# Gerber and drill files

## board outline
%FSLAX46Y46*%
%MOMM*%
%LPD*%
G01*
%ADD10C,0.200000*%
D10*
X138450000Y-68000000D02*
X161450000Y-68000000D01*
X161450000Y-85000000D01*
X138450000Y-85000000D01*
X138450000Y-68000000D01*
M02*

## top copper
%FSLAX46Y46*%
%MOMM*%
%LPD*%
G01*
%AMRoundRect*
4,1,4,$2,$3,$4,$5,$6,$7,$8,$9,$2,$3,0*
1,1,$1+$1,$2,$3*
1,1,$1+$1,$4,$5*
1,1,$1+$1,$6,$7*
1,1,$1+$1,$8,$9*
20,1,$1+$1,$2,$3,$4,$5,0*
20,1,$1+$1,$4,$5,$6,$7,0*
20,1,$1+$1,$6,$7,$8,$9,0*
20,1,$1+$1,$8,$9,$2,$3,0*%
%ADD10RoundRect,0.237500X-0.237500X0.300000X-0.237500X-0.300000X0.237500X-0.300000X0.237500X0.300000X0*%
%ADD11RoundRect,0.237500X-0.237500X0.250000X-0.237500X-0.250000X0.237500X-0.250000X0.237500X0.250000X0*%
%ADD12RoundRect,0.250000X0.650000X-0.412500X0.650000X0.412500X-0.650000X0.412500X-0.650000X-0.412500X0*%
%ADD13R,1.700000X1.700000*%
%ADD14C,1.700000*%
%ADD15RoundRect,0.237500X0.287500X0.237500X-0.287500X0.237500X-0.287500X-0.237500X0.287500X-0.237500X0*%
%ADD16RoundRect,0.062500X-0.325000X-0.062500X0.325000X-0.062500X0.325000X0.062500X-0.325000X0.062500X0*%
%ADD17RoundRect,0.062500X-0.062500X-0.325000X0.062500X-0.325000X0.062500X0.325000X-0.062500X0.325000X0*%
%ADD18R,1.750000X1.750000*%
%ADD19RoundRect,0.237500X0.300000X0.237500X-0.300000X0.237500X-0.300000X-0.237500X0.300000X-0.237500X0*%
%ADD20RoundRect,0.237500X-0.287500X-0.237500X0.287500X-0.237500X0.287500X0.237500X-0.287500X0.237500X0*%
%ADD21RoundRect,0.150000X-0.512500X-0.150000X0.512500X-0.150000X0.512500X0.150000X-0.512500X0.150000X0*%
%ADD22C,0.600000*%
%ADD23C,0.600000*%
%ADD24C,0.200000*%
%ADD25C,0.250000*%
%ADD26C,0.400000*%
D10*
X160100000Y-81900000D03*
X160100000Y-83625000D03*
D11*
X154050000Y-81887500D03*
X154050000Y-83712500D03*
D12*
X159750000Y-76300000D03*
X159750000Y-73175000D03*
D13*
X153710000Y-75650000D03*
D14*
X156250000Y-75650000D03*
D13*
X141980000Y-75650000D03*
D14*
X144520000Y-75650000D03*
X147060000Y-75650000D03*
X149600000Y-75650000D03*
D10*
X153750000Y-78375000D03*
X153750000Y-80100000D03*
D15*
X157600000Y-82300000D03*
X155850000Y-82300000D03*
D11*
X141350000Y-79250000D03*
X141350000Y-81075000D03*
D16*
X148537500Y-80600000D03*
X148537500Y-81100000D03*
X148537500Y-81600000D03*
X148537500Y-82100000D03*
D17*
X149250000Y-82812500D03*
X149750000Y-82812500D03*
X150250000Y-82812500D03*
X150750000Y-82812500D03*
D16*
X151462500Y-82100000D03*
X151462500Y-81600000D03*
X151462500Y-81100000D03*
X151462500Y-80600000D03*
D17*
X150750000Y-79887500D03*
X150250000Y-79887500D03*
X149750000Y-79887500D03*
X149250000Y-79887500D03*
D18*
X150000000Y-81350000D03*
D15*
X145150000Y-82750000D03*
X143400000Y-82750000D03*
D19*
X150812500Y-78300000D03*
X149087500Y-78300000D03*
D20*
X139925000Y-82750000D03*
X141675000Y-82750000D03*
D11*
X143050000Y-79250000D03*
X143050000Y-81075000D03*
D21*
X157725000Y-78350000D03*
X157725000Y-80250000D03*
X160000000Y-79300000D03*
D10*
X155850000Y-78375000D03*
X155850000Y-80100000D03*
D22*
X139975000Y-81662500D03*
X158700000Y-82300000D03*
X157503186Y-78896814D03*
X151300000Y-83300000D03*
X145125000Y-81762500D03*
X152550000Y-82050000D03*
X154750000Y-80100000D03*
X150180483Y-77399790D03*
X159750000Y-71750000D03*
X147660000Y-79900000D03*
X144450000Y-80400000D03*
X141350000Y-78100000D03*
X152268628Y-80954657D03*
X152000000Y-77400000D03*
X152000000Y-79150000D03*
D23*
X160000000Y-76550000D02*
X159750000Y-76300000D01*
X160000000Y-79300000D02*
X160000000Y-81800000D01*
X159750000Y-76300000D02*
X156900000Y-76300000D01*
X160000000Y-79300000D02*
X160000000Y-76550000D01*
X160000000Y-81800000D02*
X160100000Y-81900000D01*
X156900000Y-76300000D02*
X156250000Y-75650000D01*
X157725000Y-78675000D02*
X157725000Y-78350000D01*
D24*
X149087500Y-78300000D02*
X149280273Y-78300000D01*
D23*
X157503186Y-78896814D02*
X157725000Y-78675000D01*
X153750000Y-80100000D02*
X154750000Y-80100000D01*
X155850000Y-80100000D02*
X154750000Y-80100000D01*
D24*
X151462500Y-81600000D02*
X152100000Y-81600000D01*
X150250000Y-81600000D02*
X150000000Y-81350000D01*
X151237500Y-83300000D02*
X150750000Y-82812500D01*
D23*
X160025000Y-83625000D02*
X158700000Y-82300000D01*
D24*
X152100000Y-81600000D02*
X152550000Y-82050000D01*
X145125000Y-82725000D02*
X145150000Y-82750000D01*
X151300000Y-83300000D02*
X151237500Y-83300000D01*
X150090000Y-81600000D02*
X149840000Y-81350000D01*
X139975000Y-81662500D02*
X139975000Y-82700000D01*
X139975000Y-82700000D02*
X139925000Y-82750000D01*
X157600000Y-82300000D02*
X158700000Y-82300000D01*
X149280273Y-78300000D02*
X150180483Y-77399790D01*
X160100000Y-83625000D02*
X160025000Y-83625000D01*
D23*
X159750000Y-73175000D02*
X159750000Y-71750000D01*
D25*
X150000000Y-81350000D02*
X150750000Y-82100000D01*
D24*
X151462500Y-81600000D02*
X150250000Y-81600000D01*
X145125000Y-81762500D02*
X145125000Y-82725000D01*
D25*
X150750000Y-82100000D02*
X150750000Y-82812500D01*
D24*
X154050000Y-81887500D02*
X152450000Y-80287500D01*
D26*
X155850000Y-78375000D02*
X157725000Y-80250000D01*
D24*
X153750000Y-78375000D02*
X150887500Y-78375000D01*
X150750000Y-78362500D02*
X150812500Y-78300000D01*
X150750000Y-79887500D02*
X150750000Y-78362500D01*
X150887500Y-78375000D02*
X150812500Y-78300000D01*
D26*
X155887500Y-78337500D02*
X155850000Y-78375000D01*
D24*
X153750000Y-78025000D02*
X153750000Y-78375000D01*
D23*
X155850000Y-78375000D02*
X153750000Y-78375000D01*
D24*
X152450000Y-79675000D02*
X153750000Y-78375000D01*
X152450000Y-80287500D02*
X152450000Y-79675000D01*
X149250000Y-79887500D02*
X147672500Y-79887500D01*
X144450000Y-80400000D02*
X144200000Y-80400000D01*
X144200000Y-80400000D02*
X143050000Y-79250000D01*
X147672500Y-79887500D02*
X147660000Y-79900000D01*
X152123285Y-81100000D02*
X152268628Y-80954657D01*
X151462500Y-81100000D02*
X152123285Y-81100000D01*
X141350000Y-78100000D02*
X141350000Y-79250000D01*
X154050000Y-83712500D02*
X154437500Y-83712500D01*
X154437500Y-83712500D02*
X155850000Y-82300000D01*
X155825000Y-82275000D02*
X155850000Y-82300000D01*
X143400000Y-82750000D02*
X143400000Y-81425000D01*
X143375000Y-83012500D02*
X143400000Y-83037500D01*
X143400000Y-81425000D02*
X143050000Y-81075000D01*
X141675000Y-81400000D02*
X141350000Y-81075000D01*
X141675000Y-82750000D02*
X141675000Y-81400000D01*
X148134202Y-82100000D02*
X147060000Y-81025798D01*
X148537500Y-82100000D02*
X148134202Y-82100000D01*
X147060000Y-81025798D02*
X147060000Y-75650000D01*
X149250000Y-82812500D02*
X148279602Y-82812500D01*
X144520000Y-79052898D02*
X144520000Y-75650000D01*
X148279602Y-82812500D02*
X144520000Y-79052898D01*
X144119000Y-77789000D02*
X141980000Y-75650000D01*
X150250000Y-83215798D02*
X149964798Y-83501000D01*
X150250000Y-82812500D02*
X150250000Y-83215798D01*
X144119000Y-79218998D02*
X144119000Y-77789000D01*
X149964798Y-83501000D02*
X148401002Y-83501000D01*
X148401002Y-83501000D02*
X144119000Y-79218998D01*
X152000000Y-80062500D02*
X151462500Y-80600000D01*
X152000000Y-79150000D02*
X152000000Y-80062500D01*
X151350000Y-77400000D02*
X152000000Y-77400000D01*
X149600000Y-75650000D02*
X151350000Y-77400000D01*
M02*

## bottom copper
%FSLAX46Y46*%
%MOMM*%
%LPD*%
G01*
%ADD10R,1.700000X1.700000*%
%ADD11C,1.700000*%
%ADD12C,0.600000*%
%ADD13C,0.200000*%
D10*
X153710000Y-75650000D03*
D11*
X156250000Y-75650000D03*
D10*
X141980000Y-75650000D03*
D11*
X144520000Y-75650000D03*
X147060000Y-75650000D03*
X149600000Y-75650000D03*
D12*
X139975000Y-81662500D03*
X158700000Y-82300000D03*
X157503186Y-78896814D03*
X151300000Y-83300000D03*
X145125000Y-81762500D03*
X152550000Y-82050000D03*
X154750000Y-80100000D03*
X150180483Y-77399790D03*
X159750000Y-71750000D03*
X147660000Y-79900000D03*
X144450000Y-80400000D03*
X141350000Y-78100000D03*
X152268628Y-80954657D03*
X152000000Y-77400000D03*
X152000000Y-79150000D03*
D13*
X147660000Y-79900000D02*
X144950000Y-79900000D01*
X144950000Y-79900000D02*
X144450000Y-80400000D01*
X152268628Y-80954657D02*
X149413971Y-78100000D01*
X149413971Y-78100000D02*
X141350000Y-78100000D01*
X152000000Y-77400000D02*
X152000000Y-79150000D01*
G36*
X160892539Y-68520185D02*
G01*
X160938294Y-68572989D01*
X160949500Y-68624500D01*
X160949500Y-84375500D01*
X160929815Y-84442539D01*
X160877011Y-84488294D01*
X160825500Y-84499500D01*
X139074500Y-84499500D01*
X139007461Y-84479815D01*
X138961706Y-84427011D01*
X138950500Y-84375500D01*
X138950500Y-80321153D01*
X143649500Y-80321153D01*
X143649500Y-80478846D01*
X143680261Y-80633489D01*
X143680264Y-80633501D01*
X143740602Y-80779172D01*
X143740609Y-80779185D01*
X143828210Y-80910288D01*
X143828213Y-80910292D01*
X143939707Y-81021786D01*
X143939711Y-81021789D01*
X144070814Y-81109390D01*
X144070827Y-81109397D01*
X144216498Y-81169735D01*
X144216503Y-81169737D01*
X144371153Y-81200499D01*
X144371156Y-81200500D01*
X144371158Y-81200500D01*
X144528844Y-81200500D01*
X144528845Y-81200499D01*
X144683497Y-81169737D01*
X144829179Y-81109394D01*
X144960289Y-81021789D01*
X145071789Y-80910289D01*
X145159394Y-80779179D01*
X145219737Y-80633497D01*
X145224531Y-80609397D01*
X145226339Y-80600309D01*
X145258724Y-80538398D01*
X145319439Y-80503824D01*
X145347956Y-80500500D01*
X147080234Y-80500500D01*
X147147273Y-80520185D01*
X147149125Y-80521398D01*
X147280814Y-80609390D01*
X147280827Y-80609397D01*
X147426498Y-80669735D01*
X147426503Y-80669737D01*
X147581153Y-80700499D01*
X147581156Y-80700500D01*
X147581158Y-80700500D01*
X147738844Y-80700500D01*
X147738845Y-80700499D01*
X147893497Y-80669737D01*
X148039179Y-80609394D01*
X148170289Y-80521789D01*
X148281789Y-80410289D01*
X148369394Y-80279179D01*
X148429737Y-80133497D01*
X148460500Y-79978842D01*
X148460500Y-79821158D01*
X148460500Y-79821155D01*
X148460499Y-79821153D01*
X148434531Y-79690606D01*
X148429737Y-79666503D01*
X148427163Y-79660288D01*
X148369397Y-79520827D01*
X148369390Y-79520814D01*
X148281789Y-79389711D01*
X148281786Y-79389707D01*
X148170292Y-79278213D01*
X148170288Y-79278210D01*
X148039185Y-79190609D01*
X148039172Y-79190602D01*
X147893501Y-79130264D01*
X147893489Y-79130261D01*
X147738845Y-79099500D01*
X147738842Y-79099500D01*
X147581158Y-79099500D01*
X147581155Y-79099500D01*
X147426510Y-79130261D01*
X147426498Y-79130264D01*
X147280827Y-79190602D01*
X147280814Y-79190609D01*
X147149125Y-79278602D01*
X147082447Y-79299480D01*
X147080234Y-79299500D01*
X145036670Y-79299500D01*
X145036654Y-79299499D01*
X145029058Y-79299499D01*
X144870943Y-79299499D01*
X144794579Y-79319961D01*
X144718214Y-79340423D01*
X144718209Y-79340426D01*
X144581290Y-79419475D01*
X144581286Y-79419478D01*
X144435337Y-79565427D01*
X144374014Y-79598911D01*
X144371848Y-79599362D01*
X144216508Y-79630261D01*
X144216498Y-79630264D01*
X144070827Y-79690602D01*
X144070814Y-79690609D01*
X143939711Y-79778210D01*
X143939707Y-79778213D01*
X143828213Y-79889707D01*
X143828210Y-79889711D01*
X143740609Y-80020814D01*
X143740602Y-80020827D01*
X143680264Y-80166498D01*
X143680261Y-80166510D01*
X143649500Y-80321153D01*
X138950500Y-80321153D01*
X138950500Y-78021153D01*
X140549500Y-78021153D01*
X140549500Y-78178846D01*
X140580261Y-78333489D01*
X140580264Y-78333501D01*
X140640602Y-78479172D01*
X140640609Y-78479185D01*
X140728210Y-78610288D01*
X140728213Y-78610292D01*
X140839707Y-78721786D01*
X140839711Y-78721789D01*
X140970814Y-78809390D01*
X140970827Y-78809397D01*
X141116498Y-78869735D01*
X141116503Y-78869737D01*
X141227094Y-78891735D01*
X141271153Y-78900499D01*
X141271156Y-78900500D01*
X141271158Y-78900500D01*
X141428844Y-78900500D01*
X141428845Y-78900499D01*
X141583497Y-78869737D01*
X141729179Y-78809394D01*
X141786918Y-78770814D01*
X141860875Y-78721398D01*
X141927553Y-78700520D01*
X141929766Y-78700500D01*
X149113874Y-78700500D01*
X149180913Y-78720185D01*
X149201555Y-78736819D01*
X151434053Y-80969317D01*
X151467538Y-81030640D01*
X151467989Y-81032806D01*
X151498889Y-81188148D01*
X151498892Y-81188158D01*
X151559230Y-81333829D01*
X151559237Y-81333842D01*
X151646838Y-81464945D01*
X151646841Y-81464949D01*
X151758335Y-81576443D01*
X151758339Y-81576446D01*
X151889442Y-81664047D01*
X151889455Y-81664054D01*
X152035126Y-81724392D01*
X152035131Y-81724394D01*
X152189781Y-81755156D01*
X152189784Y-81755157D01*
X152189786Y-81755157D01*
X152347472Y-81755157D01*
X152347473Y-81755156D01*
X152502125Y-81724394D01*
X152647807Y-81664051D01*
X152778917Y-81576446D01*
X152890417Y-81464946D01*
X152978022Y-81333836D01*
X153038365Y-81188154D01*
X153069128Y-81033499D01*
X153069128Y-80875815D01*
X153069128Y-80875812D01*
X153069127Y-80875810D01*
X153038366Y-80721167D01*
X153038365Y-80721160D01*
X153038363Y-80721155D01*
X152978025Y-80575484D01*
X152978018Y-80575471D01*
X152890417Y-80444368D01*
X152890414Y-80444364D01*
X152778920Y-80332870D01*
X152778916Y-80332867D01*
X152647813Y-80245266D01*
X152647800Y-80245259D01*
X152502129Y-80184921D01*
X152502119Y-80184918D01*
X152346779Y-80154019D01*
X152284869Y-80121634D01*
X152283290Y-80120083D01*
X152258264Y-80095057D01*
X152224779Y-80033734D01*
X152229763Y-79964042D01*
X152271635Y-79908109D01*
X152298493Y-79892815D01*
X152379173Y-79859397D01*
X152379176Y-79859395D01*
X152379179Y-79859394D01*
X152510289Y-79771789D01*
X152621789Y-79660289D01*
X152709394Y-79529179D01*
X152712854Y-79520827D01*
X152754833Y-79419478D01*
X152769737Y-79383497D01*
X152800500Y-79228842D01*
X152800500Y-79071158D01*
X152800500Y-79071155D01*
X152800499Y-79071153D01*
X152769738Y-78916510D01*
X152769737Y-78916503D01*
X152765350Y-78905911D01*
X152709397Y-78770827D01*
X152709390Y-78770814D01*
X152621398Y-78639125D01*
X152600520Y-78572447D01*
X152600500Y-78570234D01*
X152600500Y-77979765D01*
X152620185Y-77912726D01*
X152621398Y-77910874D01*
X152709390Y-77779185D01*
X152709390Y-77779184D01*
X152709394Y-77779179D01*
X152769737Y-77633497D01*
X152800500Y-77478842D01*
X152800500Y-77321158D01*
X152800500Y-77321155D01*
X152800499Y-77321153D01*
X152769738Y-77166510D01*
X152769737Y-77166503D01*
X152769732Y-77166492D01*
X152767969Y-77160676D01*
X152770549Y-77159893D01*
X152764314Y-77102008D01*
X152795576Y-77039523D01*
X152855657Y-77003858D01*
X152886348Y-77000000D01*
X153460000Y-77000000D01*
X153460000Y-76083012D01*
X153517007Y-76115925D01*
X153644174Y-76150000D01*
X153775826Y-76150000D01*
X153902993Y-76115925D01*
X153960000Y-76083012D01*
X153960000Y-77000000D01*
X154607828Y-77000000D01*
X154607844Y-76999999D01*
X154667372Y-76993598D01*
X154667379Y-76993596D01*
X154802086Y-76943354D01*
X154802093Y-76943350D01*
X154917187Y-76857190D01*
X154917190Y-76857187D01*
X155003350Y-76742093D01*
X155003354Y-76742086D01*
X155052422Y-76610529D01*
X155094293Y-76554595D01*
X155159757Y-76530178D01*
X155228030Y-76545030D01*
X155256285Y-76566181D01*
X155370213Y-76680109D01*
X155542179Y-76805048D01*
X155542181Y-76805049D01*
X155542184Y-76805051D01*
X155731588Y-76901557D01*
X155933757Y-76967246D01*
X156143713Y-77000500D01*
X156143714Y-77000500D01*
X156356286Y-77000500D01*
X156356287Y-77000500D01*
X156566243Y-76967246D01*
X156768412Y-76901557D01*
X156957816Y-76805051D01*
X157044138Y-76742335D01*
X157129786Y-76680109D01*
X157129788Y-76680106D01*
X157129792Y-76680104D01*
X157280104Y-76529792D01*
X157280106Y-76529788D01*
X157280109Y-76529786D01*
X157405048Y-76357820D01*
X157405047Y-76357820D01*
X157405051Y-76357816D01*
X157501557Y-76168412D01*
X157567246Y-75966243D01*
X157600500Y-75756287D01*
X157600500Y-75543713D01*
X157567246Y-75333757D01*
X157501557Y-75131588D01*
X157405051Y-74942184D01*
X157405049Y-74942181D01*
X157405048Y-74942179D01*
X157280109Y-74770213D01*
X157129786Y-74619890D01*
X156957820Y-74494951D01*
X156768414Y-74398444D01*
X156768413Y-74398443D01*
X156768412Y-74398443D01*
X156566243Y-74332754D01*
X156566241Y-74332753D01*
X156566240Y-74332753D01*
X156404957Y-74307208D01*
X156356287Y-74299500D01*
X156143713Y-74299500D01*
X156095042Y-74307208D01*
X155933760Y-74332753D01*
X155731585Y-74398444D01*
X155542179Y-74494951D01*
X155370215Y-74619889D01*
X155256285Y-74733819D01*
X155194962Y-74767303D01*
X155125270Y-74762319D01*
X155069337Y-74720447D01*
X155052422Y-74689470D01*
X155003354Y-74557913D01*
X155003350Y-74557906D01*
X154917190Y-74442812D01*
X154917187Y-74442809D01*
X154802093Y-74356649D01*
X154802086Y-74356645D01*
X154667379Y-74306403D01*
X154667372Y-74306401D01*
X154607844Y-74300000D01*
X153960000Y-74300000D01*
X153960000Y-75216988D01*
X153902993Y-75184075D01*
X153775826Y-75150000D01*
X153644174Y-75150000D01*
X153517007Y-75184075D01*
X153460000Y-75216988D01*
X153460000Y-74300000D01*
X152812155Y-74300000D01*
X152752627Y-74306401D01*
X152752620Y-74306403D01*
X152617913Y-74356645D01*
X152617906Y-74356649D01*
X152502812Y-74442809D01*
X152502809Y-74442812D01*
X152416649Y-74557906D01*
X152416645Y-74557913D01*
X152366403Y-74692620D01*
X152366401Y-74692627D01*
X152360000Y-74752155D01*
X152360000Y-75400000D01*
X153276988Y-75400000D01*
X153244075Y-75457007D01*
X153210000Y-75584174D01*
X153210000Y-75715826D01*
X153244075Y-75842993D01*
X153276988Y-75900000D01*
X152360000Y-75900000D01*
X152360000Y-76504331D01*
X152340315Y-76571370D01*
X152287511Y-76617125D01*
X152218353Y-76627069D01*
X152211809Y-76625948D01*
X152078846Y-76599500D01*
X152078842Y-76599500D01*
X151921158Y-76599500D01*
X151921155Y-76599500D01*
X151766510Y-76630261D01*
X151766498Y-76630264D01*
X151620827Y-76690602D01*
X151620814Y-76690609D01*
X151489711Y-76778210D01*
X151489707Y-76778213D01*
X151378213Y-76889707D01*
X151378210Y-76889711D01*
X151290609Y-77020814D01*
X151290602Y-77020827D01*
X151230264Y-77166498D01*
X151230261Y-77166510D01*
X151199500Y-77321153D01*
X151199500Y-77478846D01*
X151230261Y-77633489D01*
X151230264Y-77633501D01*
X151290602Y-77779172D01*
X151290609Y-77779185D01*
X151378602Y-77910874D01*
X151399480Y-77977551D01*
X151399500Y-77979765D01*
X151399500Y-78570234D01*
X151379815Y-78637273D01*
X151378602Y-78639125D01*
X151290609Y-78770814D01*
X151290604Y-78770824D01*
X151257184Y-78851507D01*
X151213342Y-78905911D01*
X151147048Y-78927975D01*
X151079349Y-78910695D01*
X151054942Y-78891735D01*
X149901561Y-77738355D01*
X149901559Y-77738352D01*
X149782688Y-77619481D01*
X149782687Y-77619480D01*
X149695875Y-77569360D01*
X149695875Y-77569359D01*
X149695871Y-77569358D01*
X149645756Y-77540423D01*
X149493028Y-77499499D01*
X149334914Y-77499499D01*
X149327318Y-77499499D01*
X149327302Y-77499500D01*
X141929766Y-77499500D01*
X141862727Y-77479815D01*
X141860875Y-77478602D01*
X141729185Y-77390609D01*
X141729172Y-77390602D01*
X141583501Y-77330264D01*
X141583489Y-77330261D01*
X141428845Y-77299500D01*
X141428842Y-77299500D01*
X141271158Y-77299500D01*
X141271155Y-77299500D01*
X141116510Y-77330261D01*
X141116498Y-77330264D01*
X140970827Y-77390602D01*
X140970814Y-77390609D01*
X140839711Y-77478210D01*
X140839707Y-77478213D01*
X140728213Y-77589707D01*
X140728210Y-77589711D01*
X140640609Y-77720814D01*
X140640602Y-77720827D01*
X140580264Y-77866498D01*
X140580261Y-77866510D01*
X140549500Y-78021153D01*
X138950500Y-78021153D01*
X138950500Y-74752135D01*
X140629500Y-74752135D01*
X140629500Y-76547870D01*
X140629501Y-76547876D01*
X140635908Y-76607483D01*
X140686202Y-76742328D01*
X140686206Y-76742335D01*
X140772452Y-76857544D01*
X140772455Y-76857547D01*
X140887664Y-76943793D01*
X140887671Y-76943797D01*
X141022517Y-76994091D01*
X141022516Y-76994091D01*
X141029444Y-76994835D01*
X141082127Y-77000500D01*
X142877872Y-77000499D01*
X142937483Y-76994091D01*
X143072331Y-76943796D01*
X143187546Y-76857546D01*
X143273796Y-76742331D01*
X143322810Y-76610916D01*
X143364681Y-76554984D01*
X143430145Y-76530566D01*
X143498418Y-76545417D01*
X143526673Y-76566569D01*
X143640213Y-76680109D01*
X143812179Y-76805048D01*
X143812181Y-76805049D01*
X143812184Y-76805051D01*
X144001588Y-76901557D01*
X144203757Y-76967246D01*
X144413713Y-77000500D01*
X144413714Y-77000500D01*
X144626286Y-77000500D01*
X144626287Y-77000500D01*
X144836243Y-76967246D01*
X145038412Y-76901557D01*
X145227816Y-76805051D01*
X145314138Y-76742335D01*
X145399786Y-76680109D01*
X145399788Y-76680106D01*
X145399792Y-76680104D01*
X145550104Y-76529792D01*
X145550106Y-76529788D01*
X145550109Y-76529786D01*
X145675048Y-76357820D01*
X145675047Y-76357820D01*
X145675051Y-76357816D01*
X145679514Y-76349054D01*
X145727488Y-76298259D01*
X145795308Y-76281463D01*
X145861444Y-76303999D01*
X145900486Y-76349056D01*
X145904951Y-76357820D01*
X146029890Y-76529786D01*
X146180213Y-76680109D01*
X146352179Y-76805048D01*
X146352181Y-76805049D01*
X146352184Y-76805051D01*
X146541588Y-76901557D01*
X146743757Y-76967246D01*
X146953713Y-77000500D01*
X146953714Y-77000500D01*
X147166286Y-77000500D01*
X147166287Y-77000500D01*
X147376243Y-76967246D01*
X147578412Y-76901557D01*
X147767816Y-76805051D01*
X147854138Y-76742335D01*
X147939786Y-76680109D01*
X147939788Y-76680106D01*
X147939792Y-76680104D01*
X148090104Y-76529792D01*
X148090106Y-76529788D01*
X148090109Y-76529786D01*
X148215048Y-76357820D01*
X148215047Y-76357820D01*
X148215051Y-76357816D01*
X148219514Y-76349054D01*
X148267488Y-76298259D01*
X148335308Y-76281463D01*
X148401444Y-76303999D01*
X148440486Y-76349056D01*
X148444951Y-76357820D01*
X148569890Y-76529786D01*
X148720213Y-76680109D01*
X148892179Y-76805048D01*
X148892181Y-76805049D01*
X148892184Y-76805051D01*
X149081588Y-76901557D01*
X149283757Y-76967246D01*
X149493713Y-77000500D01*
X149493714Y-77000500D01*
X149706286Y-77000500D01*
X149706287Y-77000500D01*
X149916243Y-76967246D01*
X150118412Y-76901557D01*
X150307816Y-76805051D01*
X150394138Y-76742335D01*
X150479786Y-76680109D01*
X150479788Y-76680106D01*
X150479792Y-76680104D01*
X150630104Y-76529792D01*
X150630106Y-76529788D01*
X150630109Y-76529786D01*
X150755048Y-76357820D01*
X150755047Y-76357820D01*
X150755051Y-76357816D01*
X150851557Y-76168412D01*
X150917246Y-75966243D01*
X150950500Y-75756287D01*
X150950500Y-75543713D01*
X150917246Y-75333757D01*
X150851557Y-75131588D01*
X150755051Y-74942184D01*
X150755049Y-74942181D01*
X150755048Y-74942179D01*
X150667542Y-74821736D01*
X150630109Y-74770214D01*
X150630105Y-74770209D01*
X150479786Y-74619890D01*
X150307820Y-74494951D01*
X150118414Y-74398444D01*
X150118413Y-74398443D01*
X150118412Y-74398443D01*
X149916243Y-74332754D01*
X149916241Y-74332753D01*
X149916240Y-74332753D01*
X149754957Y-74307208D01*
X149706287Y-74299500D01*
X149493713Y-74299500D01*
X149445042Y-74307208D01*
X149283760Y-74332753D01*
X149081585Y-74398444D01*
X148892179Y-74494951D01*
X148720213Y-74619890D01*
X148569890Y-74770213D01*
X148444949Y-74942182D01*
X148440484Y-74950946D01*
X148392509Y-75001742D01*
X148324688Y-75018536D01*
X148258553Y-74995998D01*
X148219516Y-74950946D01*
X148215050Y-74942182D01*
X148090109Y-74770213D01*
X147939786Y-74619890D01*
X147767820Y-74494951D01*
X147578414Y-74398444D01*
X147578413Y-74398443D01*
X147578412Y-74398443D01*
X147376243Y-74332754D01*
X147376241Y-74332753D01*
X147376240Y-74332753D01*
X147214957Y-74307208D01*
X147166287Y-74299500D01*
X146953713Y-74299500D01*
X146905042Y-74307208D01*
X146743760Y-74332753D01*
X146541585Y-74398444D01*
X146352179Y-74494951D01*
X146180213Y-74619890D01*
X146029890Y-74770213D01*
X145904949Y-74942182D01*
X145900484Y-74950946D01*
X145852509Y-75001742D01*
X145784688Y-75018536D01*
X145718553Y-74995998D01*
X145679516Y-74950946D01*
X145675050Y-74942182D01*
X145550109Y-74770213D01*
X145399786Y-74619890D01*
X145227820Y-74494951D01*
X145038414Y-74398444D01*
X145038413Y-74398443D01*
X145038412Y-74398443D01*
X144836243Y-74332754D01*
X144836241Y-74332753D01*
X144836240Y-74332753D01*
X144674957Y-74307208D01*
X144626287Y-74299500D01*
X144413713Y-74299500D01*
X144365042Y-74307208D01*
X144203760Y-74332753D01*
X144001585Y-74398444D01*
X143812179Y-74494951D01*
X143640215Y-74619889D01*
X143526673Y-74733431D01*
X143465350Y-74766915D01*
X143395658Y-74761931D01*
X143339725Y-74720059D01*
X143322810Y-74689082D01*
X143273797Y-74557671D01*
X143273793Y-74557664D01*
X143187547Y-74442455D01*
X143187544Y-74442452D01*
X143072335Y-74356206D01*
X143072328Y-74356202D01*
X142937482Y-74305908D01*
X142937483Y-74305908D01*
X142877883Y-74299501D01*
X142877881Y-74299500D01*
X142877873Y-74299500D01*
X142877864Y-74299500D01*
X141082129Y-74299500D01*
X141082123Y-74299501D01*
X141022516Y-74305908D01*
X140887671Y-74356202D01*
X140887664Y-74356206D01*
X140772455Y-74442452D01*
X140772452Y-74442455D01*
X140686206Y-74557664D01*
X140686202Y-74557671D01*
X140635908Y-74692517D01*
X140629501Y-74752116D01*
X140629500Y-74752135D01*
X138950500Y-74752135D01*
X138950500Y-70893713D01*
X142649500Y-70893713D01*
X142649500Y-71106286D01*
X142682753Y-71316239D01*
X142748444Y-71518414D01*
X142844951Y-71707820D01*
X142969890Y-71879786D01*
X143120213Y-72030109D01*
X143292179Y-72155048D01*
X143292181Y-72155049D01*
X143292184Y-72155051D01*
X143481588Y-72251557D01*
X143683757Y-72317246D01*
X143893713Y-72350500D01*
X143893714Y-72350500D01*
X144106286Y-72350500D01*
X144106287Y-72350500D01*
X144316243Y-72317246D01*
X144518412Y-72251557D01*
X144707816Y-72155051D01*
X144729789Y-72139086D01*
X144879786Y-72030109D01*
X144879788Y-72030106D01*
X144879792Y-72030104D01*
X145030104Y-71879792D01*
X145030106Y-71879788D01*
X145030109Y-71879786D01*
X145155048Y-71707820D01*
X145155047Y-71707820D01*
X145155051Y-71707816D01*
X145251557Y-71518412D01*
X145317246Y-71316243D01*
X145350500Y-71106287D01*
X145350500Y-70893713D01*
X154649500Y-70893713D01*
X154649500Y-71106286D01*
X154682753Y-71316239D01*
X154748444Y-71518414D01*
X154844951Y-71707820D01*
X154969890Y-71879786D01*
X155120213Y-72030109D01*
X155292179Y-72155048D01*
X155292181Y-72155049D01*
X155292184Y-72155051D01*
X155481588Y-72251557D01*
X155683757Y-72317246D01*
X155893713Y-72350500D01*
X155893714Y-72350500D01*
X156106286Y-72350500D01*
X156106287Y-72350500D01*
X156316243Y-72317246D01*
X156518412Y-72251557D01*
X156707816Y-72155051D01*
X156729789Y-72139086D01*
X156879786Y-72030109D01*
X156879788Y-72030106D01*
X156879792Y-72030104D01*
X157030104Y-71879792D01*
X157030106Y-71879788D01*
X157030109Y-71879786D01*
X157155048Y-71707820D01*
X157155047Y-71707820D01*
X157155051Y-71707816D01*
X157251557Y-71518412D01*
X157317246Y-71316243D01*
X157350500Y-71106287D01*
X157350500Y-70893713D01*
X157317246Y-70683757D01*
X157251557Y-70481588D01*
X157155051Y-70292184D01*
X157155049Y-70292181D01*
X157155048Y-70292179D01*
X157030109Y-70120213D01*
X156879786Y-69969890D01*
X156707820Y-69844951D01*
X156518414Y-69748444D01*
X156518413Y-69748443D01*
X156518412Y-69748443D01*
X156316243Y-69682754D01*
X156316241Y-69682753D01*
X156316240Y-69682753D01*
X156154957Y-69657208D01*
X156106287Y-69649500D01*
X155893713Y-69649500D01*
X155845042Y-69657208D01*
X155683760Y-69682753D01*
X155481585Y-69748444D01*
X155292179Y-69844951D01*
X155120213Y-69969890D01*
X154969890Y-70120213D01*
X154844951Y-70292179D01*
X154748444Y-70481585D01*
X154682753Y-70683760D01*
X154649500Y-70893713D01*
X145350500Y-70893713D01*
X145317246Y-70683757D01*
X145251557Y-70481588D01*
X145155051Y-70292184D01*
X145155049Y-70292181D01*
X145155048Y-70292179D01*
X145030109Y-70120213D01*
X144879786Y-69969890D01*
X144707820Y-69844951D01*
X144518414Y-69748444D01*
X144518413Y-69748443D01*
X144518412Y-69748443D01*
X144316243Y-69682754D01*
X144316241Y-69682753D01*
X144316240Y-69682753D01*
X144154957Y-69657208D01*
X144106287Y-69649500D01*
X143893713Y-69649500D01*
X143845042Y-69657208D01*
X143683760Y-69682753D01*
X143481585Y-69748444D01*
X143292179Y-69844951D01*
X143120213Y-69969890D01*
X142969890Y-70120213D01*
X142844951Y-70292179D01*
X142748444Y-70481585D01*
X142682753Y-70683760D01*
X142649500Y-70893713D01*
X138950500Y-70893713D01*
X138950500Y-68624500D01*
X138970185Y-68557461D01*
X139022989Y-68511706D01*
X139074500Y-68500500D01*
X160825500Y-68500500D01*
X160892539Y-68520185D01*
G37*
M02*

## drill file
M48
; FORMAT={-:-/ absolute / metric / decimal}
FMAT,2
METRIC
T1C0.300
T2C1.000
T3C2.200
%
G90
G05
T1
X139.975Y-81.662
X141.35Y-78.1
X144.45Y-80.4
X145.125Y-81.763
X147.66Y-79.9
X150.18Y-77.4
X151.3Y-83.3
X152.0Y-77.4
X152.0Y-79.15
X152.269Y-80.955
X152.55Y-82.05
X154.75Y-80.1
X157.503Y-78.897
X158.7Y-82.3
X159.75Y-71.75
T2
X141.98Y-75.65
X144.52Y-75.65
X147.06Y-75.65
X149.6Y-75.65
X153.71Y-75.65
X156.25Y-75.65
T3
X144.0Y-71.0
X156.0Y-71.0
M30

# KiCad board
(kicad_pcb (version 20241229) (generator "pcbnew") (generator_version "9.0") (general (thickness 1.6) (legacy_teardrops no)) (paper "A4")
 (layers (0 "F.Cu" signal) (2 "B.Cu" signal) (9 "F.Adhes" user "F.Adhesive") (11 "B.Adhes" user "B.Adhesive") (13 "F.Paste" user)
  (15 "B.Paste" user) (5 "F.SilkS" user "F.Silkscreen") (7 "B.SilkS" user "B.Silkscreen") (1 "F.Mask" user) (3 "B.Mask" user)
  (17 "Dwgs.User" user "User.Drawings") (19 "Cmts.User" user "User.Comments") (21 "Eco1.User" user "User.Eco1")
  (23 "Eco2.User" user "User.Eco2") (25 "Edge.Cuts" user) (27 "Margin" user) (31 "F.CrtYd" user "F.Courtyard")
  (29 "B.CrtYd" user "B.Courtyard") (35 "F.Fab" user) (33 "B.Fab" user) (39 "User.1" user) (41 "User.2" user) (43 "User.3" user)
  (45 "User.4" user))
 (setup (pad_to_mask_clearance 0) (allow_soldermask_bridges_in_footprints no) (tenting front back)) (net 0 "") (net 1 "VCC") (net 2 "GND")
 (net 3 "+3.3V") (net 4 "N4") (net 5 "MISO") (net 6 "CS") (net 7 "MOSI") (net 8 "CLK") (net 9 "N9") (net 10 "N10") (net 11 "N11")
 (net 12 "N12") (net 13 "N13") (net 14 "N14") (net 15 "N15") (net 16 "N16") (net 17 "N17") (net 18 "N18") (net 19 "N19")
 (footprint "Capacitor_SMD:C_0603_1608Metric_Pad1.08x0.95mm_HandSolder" (layer "F.Cu") (at 160.1 82.7625 -90)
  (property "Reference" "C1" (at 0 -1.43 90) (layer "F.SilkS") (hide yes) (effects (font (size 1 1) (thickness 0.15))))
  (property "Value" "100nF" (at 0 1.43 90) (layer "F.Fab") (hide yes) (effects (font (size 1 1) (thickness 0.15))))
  (pad "1" smd roundrect (at -0.8625 0 270) (size 1.075 0.95) (layers "F.Cu" "F.Mask" "F.Paste") (roundrect_rratio 0.25) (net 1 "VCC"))
  (pad "2" smd roundrect (at 0.8625 0 270) (size 1.075 0.95) (layers "F.Cu" "F.Mask" "F.Paste") (roundrect_rratio 0.25) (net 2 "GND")))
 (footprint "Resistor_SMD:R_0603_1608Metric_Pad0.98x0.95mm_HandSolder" (layer "F.Cu") (at 154.05 82.8 -90)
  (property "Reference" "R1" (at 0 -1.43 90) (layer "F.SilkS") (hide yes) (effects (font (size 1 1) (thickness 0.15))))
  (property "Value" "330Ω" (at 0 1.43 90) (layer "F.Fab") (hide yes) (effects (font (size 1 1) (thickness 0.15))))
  (pad "1" smd roundrect (at -0.9125 0 270) (size 0.975 0.95) (layers "F.Cu" "F.Mask" "F.Paste") (roundrect_rratio 0.25) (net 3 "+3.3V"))
  (pad "2" smd roundrect (at 0.9125 0 270) (size 0.975 0.95) (layers "F.Cu" "F.Mask" "F.Paste") (roundrect_rratio 0.25) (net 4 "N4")))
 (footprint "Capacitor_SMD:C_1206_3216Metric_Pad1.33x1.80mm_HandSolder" (layer "F.Cu") (at 159.75 74.7375 90)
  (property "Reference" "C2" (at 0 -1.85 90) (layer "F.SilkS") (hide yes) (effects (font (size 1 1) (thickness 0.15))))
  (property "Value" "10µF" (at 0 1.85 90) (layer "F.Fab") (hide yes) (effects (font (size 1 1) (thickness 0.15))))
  (pad "1" smd roundrect (at -1.5625 0 90) (size 1.325 1.8) (layers "F.Cu" "F.Mask" "F.Paste") (roundrect_rratio 0.188679) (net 1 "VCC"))
  (pad "2" smd roundrect (at 1.5625 0 90) (size 1.325 1.8) (layers "F.Cu" "F.Mask" "F.Paste") (roundrect_rratio 0.188679) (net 2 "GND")))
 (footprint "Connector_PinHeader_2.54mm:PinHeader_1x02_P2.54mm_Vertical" (layer "F.Cu") (at 153.71 75.65 90)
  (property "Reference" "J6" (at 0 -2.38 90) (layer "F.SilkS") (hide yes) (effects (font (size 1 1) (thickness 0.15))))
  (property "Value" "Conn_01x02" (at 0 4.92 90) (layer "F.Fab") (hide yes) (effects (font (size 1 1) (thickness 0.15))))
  (pad "1" thru_hole rect (at 0 0 90) (size 1.7 1.7) (drill 1) (layers "*.Cu" "*.Mask") (remove_unused_layers no) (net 2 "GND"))
  (pad "2" thru_hole circle (at 0 2.54 90) (size 1.7 1.7) (drill 1) (layers "*.Cu" "*.Mask") (remove_unused_layers no) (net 1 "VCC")))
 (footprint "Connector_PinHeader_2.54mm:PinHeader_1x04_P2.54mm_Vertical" (layer "F.Cu") (at 141.98 75.65 90)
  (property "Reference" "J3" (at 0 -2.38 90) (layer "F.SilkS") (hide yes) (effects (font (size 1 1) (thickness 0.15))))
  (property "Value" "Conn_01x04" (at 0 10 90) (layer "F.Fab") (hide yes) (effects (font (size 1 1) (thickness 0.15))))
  (pad "1" thru_hole rect (at 0 0 90) (size 1.7 1.7) (drill 1) (layers "*.Cu" "*.Mask") (remove_unused_layers no) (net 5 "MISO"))
  (pad "2" thru_hole circle (at 0 2.54 90) (size 1.7 1.7) (drill 1) (layers "*.Cu" "*.Mask") (remove_unused_layers no) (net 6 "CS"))
  (pad "3" thru_hole circle (at 0 5.08 90) (size 1.7 1.7) (drill 1) (layers "*.Cu" "*.Mask") (remove_unused_layers no) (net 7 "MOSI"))
  (pad "4" thru_hole circle (at 0 7.62 90) (size 1.7 1.7) (drill 1) (layers "*.Cu" "*.Mask") (remove_unused_layers no) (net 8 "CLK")))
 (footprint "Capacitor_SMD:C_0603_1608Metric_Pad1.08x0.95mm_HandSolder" (layer "F.Cu") (at 153.75 79.2375 -90)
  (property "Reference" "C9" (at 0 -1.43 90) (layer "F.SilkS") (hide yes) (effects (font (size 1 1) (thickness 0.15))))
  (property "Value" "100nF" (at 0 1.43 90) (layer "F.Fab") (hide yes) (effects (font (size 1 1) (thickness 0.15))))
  (pad "1" smd roundrect (at -0.8625 0 270) (size 1.075 0.95) (layers "F.Cu" "F.Mask" "F.Paste") (roundrect_rratio 0.25) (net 3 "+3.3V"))
  (pad "2" smd roundrect (at 0.8625 0 270) (size 1.075 0.95) (layers "F.Cu" "F.Mask" "F.Paste") (roundrect_rratio 0.25) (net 2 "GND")))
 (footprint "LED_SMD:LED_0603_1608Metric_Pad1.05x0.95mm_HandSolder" (layer "F.Cu") (at 156.725 82.3 180)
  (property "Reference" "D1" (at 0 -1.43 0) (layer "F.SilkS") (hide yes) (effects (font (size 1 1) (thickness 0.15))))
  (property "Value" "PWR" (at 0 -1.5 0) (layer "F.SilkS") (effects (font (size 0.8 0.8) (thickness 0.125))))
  (pad "1" smd roundrect (at -0.875 0 180) (size 1.05 0.95) (layers "F.Cu" "F.Mask" "F.Paste") (roundrect_rratio 0.25) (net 2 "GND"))
  (pad "2" smd roundrect (at 0.875 0 180) (size 1.05 0.95) (layers "F.Cu" "F.Mask" "F.Paste") (roundrect_rratio 0.25) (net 4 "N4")))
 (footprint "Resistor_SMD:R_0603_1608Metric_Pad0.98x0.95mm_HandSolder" (layer "F.Cu") (at 141.35 80.1625 -90)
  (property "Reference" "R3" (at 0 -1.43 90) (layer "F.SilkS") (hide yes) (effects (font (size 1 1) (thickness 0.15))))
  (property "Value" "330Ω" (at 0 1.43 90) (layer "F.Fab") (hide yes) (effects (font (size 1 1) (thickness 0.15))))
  (pad "1" smd roundrect (at -0.9125 0 270) (size 0.975 0.95) (layers "F.Cu" "F.Mask" "F.Paste") (roundrect_rratio 0.25) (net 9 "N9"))
  (pad "2" smd roundrect (at 0.9125 0 270) (size 0.975 0.95) (layers "F.Cu" "F.Mask" "F.Paste") (roundrect_rratio 0.25) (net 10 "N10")))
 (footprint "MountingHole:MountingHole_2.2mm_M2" (layer "F.Cu") (at 144 71)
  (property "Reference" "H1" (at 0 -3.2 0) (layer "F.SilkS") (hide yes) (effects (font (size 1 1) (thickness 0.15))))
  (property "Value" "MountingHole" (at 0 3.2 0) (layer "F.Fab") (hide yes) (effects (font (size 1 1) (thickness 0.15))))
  (pad "" np_thru_hole circle (at 0 0) (size 2.2 2.2) (drill 2.2) (layers "*.Cu" "*.Mask")))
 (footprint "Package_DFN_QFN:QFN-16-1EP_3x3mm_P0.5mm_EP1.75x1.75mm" (layer "F.Cu") (at 150 81.35)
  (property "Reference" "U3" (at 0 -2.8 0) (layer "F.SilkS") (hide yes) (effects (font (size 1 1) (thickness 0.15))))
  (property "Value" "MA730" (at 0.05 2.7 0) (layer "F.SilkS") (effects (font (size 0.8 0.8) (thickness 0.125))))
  (pad "" smd roundrect (at -0.44 -0.44) (size 0.71 0.71) (layers "F.Paste") (roundrect_rratio 0.25))
  (pad "" smd roundrect (at -0.44 0.44) (size 0.71 0.71) (layers "F.Paste") (roundrect_rratio 0.25))
  (pad "" smd roundrect (at 0.44 -0.44) (size 0.71 0.71) (layers "F.Paste") (roundrect_rratio 0.25))
  (pad "" smd roundrect (at 0.44 0.44) (size 0.71 0.71) (layers "F.Paste") (roundrect_rratio 0.25))
  (pad "1" smd roundrect (at -1.4625 -0.75) (size 0.775 0.25) (layers "F.Cu" "F.Mask" "F.Paste") (roundrect_rratio 0.25) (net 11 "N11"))
  (pad "2" smd roundrect (at -1.4625 -0.25) (size 0.775 0.25) (layers "F.Cu" "F.Mask" "F.Paste") (roundrect_rratio 0.25) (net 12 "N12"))
  (pad "3" smd roundrect (at -1.4625 0.25) (size 0.775 0.25) (layers "F.Cu" "F.Mask" "F.Paste") (roundrect_rratio 0.25) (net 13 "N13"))
  (pad "4" smd roundrect (at -1.4625 0.75) (size 0.775 0.25) (layers "F.Cu" "F.Mask" "F.Paste") (roundrect_rratio 0.25) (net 7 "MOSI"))
  (pad "5" smd roundrect (at -0.75 1.4625) (size 0.25 0.775) (layers "F.Cu" "F.Mask" "F.Paste") (roundrect_rratio 0.25) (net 6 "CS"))
  (pad "6" smd roundrect (at -0.25 1.4625) (size 0.25 0.775) (layers "F.Cu" "F.Mask" "F.Paste") (roundrect_rratio 0.25) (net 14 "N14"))
  (pad "7" smd roundrect (at 0.25 1.4625) (size 0.25 0.775) (layers "F.Cu" "F.Mask" "F.Paste") (roundrect_rratio 0.25) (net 5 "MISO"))
  (pad "8" smd roundrect (at 0.75 1.4625) (size 0.25 0.775) (layers "F.Cu" "F.Mask" "F.Paste") (roundrect_rratio 0.25) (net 2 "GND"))
  (pad "9" smd roundrect (at 1.4625 0.75) (size 0.775 0.25) (layers "F.Cu" "F.Mask" "F.Paste") (roundrect_rratio 0.25) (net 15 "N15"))
  (pad "10" smd roundrect (at 1.4625 0.25) (size 0.775 0.25) (layers "F.Cu" "F.Mask" "F.Paste") (roundrect_rratio 0.25) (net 2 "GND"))
  (pad "11" smd roundrect (at 1.4625 -0.25) (size 0.775 0.25) (layers "F.Cu" "F.Mask" "F.Paste") (roundrect_rratio 0.25) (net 9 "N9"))
  (pad "12" smd roundrect (at 1.4625 -0.75) (size 0.775 0.25) (layers "F.Cu" "F.Mask" "F.Paste") (roundrect_rratio 0.25) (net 8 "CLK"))
  (pad "13" smd roundrect (at 0.75 -1.4625) (size 0.25 0.775) (layers "F.Cu" "F.Mask" "F.Paste") (roundrect_rratio 0.25) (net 3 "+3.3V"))
  (pad "14" smd roundrect (at 0.25 -1.4625) (size 0.25 0.775) (layers "F.Cu" "F.Mask" "F.Paste") (roundrect_rratio 0.25) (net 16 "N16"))
  (pad "15" smd roundrect (at -0.25 -1.4625) (size 0.25 0.775) (layers "F.Cu" "F.Mask" "F.Paste") (roundrect_rratio 0.25) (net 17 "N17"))
  (pad "16" smd roundrect (at -0.75 -1.4625) (size 0.25 0.775) (layers "F.Cu" "F.Mask" "F.Paste") (roundrect_rratio 0.25) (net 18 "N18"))
  (pad "17" smd rect (at 0 0) (size 1.75 1.75) (layers "F.Cu" "F.Mask") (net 2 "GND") (zone_connect 2)))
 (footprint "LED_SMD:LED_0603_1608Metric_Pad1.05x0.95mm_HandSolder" (layer "F.Cu") (at 144.275 82.75 180)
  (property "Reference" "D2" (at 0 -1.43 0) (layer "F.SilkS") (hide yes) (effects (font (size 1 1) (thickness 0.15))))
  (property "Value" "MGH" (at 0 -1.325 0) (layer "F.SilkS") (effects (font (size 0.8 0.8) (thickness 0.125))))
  (pad "1" smd roundrect (at -0.875 0 180) (size 1.05 0.95) (layers "F.Cu" "F.Mask" "F.Paste") (roundrect_rratio 0.25) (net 2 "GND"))
  (pad "2" smd roundrect (at 0.875 0 180) (size 1.05 0.95) (layers "F.Cu" "F.Mask" "F.Paste") (roundrect_rratio 0.25) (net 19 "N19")))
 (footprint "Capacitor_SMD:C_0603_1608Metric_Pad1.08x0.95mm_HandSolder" (layer "F.Cu") (at 149.95 78.3 180)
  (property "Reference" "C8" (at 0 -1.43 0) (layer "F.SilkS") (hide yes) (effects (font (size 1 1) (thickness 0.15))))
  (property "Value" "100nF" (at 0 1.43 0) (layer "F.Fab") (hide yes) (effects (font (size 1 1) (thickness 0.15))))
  (pad "1" smd roundrect (at -0.8625 0 180) (size 1.075 0.95) (layers "F.Cu" "F.Mask" "F.Paste") (roundrect_rratio 0.25) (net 3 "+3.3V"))
  (pad "2" smd roundrect (at 0.8625 0 180) (size 1.075 0.95) (layers "F.Cu" "F.Mask" "F.Paste") (roundrect_rratio 0.25) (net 2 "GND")))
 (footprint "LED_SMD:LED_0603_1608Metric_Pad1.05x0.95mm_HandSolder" (layer "F.Cu") (at 140.8 82.75)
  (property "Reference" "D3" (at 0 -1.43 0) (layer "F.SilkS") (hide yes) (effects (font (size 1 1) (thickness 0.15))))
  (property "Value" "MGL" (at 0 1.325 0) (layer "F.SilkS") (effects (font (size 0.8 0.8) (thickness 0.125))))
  (pad "1" smd roundrect (at -0.875 0) (size 1.05 0.95) (layers "F.Cu" "F.Mask" "F.Paste") (roundrect_rratio 0.25) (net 2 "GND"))
  (pad "2" smd roundrect (at 0.875 0) (size 1.05 0.95) (layers "F.Cu" "F.Mask" "F.Paste") (roundrect_rratio 0.25) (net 10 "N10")))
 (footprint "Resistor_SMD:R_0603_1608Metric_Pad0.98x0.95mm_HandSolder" (layer "F.Cu") (at 143.05 80.1625 -90)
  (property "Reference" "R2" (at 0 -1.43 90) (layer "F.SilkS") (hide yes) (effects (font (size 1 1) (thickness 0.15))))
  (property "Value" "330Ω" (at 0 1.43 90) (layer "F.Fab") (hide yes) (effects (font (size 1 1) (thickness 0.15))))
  (pad "1" smd roundrect (at -0.9125 0 270) (size 0.975 0.95) (layers "F.Cu" "F.Mask" "F.Paste") (roundrect_rratio 0.25) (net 18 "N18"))
  (pad "2" smd roundrect (at 0.9125 0 270) (size 0.975 0.95) (layers "F.Cu" "F.Mask" "F.Paste") (roundrect_rratio 0.25) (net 19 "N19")))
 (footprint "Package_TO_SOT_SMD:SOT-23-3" (layer "F.Cu") (at 158.8625 79.3)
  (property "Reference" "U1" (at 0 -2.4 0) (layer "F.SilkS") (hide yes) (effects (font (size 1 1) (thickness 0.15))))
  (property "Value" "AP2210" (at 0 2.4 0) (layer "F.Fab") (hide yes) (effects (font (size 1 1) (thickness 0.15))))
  (pad "1" smd roundrect (at -1.1375 -0.95) (size 1.325 0.6) (layers "F.Cu" "F.Mask" "F.Paste") (roundrect_rratio 0.25) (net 2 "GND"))
  (pad "2" smd roundrect (at -1.1375 0.95) (size 1.325 0.6) (layers "F.Cu" "F.Mask" "F.Paste") (roundrect_rratio 0.25) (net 3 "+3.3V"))
  (pad "3" smd roundrect (at 1.1375 0) (size 1.325 0.6) (layers "F.Cu" "F.Mask" "F.Paste") (roundrect_rratio 0.25) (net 1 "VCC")))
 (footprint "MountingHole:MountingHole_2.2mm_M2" (layer "F.Cu") (at 156 71)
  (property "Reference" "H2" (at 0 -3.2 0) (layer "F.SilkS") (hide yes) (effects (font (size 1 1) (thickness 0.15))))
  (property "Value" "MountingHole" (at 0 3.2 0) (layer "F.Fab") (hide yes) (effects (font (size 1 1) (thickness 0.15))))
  (pad "" np_thru_hole circle (at 0 0) (size 2.2 2.2) (drill 2.2) (layers "*.Cu" "*.Mask")))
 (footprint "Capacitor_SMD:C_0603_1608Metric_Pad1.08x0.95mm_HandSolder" (layer "F.Cu") (at 155.85 79.2375 -90)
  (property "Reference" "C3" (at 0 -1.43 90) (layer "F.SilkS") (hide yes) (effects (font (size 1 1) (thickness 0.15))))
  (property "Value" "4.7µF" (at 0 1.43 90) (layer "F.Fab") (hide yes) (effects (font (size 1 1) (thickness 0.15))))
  (pad "1" smd roundrect (at -0.8625 0 270) (size 1.075 0.95) (layers "F.Cu" "F.Mask" "F.Paste") (roundrect_rratio 0.25) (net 3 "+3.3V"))
  (pad "2" smd roundrect (at 0.8625 0 270) (size 1.075 0.95) (layers "F.Cu" "F.Mask" "F.Paste") (roundrect_rratio 0.25) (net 2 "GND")))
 (gr_rect (start 138.45 68) (end 161.45 85) (stroke (width 0.2) (type solid)) (fill no) (layer "Edge.Cuts"))
 (segment (start 160 76.55) (end 159.75 76.3) (width 0.6) (layer "F.Cu") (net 1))
 (segment (start 160 79.3) (end 160 81.8) (width 0.6) (layer "F.Cu") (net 1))
 (segment (start 159.75 76.3) (end 156.9 76.3) (width 0.6) (layer "F.Cu") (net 1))
 (segment (start 160 79.3) (end 160 76.55) (width 0.6) (layer "F.Cu") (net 1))
 (segment (start 160 81.8) (end 160.1 81.9) (width 0.6) (layer "F.Cu") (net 1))
 (segment (start 156.9 76.3) (end 156.25 75.65) (width 0.6) (layer "F.Cu") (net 1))
 (segment (start 157.725 78.675) (end 157.725 78.35) (width 0.6) (layer "F.Cu") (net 2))
 (segment (start 149.0875 78.3) (end 149.280273 78.3) (width 0.2) (layer "F.Cu") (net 2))
 (segment (start 157.503186 78.896814) (end 157.725 78.675) (width 0.6) (layer "F.Cu") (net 2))
 (segment (start 153.75 80.1) (end 154.75 80.1) (width 0.6) (layer "F.Cu") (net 2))
 (segment (start 155.85 80.1) (end 154.75 80.1) (width 0.6) (layer "F.Cu") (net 2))
 (segment (start 151.4625 81.6) (end 152.1 81.6) (width 0.2) (layer "F.Cu") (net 2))
 (segment (start 150.25 81.6) (end 150 81.35) (width 0.2) (layer "F.Cu") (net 2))
 (segment (start 151.2375 83.3) (end 150.75 82.8125) (width 0.2) (layer "F.Cu") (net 2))
 (segment (start 160.025 83.625) (end 158.7 82.3) (width 0.6) (layer "F.Cu") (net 2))
 (segment (start 152.1 81.6) (end 152.55 82.05) (width 0.2) (layer "F.Cu") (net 2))
 (segment (start 145.125 82.725) (end 145.15 82.75) (width 0.2) (layer "F.Cu") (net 2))
 (segment (start 151.3 83.3) (end 151.2375 83.3) (width 0.2) (layer "F.Cu") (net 2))
 (segment (start 150.09 81.6) (end 149.84 81.35) (width 0.2) (layer "F.Cu") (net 2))
 (segment (start 139.975 81.6625) (end 139.975 82.7) (width 0.2) (layer "F.Cu") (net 2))
 (segment (start 139.975 82.7) (end 139.925 82.75) (width 0.2) (layer "F.Cu") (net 2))
 (segment (start 157.6 82.3) (end 158.7 82.3) (width 0.2) (layer "F.Cu") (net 2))
 (segment (start 149.280273 78.3) (end 150.180483 77.39979) (width 0.2) (layer "F.Cu") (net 2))
 (segment (start 160.1 83.625) (end 160.025 83.625) (width 0.2) (layer "F.Cu") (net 2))
 (segment (start 159.75 73.175) (end 159.75 71.75) (width 0.6) (layer "F.Cu") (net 2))
 (segment (start 150 81.35) (end 150.75 82.1) (width 0.25) (layer "F.Cu") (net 2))
 (segment (start 151.4625 81.6) (end 150.25 81.6) (width 0.2) (layer "F.Cu") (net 2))
 (segment (start 145.125 81.7625) (end 145.125 82.725) (width 0.2) (layer "F.Cu") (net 2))
 (segment (start 150.75 82.1) (end 150.75 82.8125) (width 0.25) (layer "F.Cu") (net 2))
 (via (at 139.975 81.6625) (size 0.6) (drill 0.3) (layers "F.Cu" "B.Cu") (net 2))
 (via (at 158.7 82.3) (size 0.6) (drill 0.3) (layers "F.Cu" "B.Cu") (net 2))
 (via (at 157.503186 78.896814) (size 0.6) (drill 0.3) (layers "F.Cu" "B.Cu") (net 2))
 (via (at 151.3 83.3) (size 0.6) (drill 0.3) (layers "F.Cu" "B.Cu") (free yes) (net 2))
 (via (at 145.125 81.7625) (size 0.6) (drill 0.3) (layers "F.Cu" "B.Cu") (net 2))
 (via (at 152.55 82.05) (size 0.6) (drill 0.3) (layers "F.Cu" "B.Cu") (free yes) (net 2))
 (via (at 154.75 80.1) (size 0.6) (drill 0.3) (layers "F.Cu" "B.Cu") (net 2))
 (via (at 150.180483 77.39979) (size 0.6) (drill 0.3) (layers "F.Cu" "B.Cu") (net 2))
 (via (at 159.75 71.75) (size 0.6) (drill 0.3) (layers "F.Cu" "B.Cu") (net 2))
 (segment (start 154.05 81.8875) (end 152.45 80.2875) (width 0.2) (layer "F.Cu") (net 3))
 (segment (start 155.85 78.375) (end 157.725 80.25) (width 0.4) (layer "F.Cu") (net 3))
 (segment (start 153.75 78.375) (end 150.8875 78.375) (width 0.2) (layer "F.Cu") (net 3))
 (segment (start 150.75 78.3625) (end 150.8125 78.3) (width 0.2) (layer "F.Cu") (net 3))
 (segment (start 150.75 79.8875) (end 150.75 78.3625) (width 0.2) (layer "F.Cu") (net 3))
 (segment (start 150.8875 78.375) (end 150.8125 78.3) (width 0.2) (layer "F.Cu") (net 3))
 (segment (start 155.8875 78.3375) (end 155.85 78.375) (width 0.4) (layer "F.Cu") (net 3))
 (segment (start 153.75 78.025) (end 153.75 78.375) (width 0.2) (layer "F.Cu") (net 3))
 (segment (start 155.85 78.375) (end 153.75 78.375) (width 0.6) (layer "F.Cu") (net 3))
 (segment (start 152.45 79.675) (end 153.75 78.375) (width 0.2) (layer "F.Cu") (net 3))
 (segment (start 152.45 80.2875) (end 152.45 79.675) (width 0.2) (layer "F.Cu") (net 3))
 (segment (start 149.25 79.8875) (end 147.6725 79.8875) (width 0.2) (layer "F.Cu") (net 18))
 (segment (start 144.45 80.4) (end 144.2 80.4) (width 0.2) (layer "F.Cu") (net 18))
 (segment (start 144.2 80.4) (end 143.05 79.25) (width 0.2) (layer "F.Cu") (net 18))
 (segment (start 147.6725 79.8875) (end 147.66 79.9) (width 0.2) (layer "F.Cu") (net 18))
 (via (at 147.66 79.9) (size 0.6) (drill 0.3) (layers "F.Cu" "B.Cu") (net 18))
 (via (at 144.45 80.4) (size 0.6) (drill 0.3) (layers "F.Cu" "B.Cu") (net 18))
 (segment (start 147.66 79.9) (end 144.95 79.9) (width 0.2) (layer "B.Cu") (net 18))
 (segment (start 144.95 79.9) (end 144.45 80.4) (width 0.2) (layer "B.Cu") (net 18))
 (segment (start 152.123285 81.1) (end 152.268628 80.954657) (width 0.2) (layer "F.Cu") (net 9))
 (segment (start 151.4625 81.1) (end 152.123285 81.1) (width 0.2) (layer "F.Cu") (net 9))
 (segment (start 141.35 78.1) (end 141.35 79.25) (width 0.2) (layer "F.Cu") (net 9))
 (via (at 141.35 78.1) (size 0.6) (drill 0.3) (layers "F.Cu" "B.Cu") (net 9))
 (via (at 152.268628 80.954657) (size 0.6) (drill 0.3) (layers "F.Cu" "B.Cu") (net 9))
 (segment (start 152.268628 80.954657) (end 149.413971 78.1) (width 0.2) (layer "B.Cu") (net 9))
 (segment (start 149.413971 78.1) (end 141.35 78.1) (width 0.2) (layer "B.Cu") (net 9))
 (segment (start 154.05 83.7125) (end 154.4375 83.7125) (width 0.2) (layer "F.Cu") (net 4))
 (segment (start 154.4375 83.7125) (end 155.85 82.3) (width 0.2) (layer "F.Cu") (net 4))
 (segment (start 155.825 82.275) (end 155.85 82.3) (width 0.2) (layer "F.Cu") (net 4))
 (segment (start 143.4 82.75) (end 143.4 81.425) (width 0.2) (layer "F.Cu") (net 19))
 (segment (start 143.375 83.0125) (end 143.4 83.0375) (width 0.2) (layer "F.Cu") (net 19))
 (segment (start 143.4 81.425) (end 143.05 81.075) (width 0.2) (layer "F.Cu") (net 19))
 (segment (start 141.675 81.4) (end 141.35 81.075) (width 0.2) (layer "F.Cu") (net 10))
 (segment (start 141.675 82.75) (end 141.675 81.4) (width 0.2) (layer "F.Cu") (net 10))
 (segment (start 148.134202 82.1) (end 147.06 81.025798) (width 0.2) (layer "F.Cu") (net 7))
 (segment (start 148.5375 82.1) (end 148.134202 82.1) (width 0.2) (layer "F.Cu") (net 7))
 (segment (start 147.06 81.025798) (end 147.06 75.65) (width 0.2) (layer "F.Cu") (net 7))
 (segment (start 149.25 82.8125) (end 148.279602 82.8125) (width 0.2) (layer "F.Cu") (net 6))
 (segment (start 144.52 79.052898) (end 144.52 75.65) (width 0.2) (layer "F.Cu") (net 6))
 (segment (start 148.279602 82.8125) (end 144.52 79.052898) (width 0.2) (layer "F.Cu") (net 6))
 (segment (start 144.119 77.789) (end 141.98 75.65) (width 0.2) (layer "F.Cu") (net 5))
 (segment (start 150.25 83.215798) (end 149.964798 83.501) (width 0.2) (layer "F.Cu") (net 5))
 (segment (start 150.25 82.8125) (end 150.25 83.215798) (width 0.2) (layer "F.Cu") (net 5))
 (segment (start 144.119 79.218998) (end 144.119 77.789) (width 0.2) (layer "F.Cu") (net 5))
 (segment (start 149.964798 83.501) (end 148.401002 83.501) (width 0.2) (layer "F.Cu") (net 5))
 (segment (start 148.401002 83.501) (end 144.119 79.218998) (width 0.2) (layer "F.Cu") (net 5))
 (segment (start 152 80.0625) (end 151.4625 80.6) (width 0.2) (layer "F.Cu") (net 8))
 (segment (start 152 79.15) (end 152 80.0625) (width 0.2) (layer "F.Cu") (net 8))
 (segment (start 151.35 77.4) (end 152 77.4) (width 0.2) (layer "F.Cu") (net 8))
 (segment (start 149.6 75.65) (end 151.35 77.4) (width 0.2) (layer "F.Cu") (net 8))
 (via (at 152 77.4) (size 0.6) (drill 0.3) (layers "F.Cu" "B.Cu") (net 8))
 (via (at 152 79.15) (size 0.6) (drill 0.3) (layers "F.Cu" "B.Cu") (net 8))
 (segment (start 152 77.4) (end 152 79.15) (width 0.2) (layer "B.Cu") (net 8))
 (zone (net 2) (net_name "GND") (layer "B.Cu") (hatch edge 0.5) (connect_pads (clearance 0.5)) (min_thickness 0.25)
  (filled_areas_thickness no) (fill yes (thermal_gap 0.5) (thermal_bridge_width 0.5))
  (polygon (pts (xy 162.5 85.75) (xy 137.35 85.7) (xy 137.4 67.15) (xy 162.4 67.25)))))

